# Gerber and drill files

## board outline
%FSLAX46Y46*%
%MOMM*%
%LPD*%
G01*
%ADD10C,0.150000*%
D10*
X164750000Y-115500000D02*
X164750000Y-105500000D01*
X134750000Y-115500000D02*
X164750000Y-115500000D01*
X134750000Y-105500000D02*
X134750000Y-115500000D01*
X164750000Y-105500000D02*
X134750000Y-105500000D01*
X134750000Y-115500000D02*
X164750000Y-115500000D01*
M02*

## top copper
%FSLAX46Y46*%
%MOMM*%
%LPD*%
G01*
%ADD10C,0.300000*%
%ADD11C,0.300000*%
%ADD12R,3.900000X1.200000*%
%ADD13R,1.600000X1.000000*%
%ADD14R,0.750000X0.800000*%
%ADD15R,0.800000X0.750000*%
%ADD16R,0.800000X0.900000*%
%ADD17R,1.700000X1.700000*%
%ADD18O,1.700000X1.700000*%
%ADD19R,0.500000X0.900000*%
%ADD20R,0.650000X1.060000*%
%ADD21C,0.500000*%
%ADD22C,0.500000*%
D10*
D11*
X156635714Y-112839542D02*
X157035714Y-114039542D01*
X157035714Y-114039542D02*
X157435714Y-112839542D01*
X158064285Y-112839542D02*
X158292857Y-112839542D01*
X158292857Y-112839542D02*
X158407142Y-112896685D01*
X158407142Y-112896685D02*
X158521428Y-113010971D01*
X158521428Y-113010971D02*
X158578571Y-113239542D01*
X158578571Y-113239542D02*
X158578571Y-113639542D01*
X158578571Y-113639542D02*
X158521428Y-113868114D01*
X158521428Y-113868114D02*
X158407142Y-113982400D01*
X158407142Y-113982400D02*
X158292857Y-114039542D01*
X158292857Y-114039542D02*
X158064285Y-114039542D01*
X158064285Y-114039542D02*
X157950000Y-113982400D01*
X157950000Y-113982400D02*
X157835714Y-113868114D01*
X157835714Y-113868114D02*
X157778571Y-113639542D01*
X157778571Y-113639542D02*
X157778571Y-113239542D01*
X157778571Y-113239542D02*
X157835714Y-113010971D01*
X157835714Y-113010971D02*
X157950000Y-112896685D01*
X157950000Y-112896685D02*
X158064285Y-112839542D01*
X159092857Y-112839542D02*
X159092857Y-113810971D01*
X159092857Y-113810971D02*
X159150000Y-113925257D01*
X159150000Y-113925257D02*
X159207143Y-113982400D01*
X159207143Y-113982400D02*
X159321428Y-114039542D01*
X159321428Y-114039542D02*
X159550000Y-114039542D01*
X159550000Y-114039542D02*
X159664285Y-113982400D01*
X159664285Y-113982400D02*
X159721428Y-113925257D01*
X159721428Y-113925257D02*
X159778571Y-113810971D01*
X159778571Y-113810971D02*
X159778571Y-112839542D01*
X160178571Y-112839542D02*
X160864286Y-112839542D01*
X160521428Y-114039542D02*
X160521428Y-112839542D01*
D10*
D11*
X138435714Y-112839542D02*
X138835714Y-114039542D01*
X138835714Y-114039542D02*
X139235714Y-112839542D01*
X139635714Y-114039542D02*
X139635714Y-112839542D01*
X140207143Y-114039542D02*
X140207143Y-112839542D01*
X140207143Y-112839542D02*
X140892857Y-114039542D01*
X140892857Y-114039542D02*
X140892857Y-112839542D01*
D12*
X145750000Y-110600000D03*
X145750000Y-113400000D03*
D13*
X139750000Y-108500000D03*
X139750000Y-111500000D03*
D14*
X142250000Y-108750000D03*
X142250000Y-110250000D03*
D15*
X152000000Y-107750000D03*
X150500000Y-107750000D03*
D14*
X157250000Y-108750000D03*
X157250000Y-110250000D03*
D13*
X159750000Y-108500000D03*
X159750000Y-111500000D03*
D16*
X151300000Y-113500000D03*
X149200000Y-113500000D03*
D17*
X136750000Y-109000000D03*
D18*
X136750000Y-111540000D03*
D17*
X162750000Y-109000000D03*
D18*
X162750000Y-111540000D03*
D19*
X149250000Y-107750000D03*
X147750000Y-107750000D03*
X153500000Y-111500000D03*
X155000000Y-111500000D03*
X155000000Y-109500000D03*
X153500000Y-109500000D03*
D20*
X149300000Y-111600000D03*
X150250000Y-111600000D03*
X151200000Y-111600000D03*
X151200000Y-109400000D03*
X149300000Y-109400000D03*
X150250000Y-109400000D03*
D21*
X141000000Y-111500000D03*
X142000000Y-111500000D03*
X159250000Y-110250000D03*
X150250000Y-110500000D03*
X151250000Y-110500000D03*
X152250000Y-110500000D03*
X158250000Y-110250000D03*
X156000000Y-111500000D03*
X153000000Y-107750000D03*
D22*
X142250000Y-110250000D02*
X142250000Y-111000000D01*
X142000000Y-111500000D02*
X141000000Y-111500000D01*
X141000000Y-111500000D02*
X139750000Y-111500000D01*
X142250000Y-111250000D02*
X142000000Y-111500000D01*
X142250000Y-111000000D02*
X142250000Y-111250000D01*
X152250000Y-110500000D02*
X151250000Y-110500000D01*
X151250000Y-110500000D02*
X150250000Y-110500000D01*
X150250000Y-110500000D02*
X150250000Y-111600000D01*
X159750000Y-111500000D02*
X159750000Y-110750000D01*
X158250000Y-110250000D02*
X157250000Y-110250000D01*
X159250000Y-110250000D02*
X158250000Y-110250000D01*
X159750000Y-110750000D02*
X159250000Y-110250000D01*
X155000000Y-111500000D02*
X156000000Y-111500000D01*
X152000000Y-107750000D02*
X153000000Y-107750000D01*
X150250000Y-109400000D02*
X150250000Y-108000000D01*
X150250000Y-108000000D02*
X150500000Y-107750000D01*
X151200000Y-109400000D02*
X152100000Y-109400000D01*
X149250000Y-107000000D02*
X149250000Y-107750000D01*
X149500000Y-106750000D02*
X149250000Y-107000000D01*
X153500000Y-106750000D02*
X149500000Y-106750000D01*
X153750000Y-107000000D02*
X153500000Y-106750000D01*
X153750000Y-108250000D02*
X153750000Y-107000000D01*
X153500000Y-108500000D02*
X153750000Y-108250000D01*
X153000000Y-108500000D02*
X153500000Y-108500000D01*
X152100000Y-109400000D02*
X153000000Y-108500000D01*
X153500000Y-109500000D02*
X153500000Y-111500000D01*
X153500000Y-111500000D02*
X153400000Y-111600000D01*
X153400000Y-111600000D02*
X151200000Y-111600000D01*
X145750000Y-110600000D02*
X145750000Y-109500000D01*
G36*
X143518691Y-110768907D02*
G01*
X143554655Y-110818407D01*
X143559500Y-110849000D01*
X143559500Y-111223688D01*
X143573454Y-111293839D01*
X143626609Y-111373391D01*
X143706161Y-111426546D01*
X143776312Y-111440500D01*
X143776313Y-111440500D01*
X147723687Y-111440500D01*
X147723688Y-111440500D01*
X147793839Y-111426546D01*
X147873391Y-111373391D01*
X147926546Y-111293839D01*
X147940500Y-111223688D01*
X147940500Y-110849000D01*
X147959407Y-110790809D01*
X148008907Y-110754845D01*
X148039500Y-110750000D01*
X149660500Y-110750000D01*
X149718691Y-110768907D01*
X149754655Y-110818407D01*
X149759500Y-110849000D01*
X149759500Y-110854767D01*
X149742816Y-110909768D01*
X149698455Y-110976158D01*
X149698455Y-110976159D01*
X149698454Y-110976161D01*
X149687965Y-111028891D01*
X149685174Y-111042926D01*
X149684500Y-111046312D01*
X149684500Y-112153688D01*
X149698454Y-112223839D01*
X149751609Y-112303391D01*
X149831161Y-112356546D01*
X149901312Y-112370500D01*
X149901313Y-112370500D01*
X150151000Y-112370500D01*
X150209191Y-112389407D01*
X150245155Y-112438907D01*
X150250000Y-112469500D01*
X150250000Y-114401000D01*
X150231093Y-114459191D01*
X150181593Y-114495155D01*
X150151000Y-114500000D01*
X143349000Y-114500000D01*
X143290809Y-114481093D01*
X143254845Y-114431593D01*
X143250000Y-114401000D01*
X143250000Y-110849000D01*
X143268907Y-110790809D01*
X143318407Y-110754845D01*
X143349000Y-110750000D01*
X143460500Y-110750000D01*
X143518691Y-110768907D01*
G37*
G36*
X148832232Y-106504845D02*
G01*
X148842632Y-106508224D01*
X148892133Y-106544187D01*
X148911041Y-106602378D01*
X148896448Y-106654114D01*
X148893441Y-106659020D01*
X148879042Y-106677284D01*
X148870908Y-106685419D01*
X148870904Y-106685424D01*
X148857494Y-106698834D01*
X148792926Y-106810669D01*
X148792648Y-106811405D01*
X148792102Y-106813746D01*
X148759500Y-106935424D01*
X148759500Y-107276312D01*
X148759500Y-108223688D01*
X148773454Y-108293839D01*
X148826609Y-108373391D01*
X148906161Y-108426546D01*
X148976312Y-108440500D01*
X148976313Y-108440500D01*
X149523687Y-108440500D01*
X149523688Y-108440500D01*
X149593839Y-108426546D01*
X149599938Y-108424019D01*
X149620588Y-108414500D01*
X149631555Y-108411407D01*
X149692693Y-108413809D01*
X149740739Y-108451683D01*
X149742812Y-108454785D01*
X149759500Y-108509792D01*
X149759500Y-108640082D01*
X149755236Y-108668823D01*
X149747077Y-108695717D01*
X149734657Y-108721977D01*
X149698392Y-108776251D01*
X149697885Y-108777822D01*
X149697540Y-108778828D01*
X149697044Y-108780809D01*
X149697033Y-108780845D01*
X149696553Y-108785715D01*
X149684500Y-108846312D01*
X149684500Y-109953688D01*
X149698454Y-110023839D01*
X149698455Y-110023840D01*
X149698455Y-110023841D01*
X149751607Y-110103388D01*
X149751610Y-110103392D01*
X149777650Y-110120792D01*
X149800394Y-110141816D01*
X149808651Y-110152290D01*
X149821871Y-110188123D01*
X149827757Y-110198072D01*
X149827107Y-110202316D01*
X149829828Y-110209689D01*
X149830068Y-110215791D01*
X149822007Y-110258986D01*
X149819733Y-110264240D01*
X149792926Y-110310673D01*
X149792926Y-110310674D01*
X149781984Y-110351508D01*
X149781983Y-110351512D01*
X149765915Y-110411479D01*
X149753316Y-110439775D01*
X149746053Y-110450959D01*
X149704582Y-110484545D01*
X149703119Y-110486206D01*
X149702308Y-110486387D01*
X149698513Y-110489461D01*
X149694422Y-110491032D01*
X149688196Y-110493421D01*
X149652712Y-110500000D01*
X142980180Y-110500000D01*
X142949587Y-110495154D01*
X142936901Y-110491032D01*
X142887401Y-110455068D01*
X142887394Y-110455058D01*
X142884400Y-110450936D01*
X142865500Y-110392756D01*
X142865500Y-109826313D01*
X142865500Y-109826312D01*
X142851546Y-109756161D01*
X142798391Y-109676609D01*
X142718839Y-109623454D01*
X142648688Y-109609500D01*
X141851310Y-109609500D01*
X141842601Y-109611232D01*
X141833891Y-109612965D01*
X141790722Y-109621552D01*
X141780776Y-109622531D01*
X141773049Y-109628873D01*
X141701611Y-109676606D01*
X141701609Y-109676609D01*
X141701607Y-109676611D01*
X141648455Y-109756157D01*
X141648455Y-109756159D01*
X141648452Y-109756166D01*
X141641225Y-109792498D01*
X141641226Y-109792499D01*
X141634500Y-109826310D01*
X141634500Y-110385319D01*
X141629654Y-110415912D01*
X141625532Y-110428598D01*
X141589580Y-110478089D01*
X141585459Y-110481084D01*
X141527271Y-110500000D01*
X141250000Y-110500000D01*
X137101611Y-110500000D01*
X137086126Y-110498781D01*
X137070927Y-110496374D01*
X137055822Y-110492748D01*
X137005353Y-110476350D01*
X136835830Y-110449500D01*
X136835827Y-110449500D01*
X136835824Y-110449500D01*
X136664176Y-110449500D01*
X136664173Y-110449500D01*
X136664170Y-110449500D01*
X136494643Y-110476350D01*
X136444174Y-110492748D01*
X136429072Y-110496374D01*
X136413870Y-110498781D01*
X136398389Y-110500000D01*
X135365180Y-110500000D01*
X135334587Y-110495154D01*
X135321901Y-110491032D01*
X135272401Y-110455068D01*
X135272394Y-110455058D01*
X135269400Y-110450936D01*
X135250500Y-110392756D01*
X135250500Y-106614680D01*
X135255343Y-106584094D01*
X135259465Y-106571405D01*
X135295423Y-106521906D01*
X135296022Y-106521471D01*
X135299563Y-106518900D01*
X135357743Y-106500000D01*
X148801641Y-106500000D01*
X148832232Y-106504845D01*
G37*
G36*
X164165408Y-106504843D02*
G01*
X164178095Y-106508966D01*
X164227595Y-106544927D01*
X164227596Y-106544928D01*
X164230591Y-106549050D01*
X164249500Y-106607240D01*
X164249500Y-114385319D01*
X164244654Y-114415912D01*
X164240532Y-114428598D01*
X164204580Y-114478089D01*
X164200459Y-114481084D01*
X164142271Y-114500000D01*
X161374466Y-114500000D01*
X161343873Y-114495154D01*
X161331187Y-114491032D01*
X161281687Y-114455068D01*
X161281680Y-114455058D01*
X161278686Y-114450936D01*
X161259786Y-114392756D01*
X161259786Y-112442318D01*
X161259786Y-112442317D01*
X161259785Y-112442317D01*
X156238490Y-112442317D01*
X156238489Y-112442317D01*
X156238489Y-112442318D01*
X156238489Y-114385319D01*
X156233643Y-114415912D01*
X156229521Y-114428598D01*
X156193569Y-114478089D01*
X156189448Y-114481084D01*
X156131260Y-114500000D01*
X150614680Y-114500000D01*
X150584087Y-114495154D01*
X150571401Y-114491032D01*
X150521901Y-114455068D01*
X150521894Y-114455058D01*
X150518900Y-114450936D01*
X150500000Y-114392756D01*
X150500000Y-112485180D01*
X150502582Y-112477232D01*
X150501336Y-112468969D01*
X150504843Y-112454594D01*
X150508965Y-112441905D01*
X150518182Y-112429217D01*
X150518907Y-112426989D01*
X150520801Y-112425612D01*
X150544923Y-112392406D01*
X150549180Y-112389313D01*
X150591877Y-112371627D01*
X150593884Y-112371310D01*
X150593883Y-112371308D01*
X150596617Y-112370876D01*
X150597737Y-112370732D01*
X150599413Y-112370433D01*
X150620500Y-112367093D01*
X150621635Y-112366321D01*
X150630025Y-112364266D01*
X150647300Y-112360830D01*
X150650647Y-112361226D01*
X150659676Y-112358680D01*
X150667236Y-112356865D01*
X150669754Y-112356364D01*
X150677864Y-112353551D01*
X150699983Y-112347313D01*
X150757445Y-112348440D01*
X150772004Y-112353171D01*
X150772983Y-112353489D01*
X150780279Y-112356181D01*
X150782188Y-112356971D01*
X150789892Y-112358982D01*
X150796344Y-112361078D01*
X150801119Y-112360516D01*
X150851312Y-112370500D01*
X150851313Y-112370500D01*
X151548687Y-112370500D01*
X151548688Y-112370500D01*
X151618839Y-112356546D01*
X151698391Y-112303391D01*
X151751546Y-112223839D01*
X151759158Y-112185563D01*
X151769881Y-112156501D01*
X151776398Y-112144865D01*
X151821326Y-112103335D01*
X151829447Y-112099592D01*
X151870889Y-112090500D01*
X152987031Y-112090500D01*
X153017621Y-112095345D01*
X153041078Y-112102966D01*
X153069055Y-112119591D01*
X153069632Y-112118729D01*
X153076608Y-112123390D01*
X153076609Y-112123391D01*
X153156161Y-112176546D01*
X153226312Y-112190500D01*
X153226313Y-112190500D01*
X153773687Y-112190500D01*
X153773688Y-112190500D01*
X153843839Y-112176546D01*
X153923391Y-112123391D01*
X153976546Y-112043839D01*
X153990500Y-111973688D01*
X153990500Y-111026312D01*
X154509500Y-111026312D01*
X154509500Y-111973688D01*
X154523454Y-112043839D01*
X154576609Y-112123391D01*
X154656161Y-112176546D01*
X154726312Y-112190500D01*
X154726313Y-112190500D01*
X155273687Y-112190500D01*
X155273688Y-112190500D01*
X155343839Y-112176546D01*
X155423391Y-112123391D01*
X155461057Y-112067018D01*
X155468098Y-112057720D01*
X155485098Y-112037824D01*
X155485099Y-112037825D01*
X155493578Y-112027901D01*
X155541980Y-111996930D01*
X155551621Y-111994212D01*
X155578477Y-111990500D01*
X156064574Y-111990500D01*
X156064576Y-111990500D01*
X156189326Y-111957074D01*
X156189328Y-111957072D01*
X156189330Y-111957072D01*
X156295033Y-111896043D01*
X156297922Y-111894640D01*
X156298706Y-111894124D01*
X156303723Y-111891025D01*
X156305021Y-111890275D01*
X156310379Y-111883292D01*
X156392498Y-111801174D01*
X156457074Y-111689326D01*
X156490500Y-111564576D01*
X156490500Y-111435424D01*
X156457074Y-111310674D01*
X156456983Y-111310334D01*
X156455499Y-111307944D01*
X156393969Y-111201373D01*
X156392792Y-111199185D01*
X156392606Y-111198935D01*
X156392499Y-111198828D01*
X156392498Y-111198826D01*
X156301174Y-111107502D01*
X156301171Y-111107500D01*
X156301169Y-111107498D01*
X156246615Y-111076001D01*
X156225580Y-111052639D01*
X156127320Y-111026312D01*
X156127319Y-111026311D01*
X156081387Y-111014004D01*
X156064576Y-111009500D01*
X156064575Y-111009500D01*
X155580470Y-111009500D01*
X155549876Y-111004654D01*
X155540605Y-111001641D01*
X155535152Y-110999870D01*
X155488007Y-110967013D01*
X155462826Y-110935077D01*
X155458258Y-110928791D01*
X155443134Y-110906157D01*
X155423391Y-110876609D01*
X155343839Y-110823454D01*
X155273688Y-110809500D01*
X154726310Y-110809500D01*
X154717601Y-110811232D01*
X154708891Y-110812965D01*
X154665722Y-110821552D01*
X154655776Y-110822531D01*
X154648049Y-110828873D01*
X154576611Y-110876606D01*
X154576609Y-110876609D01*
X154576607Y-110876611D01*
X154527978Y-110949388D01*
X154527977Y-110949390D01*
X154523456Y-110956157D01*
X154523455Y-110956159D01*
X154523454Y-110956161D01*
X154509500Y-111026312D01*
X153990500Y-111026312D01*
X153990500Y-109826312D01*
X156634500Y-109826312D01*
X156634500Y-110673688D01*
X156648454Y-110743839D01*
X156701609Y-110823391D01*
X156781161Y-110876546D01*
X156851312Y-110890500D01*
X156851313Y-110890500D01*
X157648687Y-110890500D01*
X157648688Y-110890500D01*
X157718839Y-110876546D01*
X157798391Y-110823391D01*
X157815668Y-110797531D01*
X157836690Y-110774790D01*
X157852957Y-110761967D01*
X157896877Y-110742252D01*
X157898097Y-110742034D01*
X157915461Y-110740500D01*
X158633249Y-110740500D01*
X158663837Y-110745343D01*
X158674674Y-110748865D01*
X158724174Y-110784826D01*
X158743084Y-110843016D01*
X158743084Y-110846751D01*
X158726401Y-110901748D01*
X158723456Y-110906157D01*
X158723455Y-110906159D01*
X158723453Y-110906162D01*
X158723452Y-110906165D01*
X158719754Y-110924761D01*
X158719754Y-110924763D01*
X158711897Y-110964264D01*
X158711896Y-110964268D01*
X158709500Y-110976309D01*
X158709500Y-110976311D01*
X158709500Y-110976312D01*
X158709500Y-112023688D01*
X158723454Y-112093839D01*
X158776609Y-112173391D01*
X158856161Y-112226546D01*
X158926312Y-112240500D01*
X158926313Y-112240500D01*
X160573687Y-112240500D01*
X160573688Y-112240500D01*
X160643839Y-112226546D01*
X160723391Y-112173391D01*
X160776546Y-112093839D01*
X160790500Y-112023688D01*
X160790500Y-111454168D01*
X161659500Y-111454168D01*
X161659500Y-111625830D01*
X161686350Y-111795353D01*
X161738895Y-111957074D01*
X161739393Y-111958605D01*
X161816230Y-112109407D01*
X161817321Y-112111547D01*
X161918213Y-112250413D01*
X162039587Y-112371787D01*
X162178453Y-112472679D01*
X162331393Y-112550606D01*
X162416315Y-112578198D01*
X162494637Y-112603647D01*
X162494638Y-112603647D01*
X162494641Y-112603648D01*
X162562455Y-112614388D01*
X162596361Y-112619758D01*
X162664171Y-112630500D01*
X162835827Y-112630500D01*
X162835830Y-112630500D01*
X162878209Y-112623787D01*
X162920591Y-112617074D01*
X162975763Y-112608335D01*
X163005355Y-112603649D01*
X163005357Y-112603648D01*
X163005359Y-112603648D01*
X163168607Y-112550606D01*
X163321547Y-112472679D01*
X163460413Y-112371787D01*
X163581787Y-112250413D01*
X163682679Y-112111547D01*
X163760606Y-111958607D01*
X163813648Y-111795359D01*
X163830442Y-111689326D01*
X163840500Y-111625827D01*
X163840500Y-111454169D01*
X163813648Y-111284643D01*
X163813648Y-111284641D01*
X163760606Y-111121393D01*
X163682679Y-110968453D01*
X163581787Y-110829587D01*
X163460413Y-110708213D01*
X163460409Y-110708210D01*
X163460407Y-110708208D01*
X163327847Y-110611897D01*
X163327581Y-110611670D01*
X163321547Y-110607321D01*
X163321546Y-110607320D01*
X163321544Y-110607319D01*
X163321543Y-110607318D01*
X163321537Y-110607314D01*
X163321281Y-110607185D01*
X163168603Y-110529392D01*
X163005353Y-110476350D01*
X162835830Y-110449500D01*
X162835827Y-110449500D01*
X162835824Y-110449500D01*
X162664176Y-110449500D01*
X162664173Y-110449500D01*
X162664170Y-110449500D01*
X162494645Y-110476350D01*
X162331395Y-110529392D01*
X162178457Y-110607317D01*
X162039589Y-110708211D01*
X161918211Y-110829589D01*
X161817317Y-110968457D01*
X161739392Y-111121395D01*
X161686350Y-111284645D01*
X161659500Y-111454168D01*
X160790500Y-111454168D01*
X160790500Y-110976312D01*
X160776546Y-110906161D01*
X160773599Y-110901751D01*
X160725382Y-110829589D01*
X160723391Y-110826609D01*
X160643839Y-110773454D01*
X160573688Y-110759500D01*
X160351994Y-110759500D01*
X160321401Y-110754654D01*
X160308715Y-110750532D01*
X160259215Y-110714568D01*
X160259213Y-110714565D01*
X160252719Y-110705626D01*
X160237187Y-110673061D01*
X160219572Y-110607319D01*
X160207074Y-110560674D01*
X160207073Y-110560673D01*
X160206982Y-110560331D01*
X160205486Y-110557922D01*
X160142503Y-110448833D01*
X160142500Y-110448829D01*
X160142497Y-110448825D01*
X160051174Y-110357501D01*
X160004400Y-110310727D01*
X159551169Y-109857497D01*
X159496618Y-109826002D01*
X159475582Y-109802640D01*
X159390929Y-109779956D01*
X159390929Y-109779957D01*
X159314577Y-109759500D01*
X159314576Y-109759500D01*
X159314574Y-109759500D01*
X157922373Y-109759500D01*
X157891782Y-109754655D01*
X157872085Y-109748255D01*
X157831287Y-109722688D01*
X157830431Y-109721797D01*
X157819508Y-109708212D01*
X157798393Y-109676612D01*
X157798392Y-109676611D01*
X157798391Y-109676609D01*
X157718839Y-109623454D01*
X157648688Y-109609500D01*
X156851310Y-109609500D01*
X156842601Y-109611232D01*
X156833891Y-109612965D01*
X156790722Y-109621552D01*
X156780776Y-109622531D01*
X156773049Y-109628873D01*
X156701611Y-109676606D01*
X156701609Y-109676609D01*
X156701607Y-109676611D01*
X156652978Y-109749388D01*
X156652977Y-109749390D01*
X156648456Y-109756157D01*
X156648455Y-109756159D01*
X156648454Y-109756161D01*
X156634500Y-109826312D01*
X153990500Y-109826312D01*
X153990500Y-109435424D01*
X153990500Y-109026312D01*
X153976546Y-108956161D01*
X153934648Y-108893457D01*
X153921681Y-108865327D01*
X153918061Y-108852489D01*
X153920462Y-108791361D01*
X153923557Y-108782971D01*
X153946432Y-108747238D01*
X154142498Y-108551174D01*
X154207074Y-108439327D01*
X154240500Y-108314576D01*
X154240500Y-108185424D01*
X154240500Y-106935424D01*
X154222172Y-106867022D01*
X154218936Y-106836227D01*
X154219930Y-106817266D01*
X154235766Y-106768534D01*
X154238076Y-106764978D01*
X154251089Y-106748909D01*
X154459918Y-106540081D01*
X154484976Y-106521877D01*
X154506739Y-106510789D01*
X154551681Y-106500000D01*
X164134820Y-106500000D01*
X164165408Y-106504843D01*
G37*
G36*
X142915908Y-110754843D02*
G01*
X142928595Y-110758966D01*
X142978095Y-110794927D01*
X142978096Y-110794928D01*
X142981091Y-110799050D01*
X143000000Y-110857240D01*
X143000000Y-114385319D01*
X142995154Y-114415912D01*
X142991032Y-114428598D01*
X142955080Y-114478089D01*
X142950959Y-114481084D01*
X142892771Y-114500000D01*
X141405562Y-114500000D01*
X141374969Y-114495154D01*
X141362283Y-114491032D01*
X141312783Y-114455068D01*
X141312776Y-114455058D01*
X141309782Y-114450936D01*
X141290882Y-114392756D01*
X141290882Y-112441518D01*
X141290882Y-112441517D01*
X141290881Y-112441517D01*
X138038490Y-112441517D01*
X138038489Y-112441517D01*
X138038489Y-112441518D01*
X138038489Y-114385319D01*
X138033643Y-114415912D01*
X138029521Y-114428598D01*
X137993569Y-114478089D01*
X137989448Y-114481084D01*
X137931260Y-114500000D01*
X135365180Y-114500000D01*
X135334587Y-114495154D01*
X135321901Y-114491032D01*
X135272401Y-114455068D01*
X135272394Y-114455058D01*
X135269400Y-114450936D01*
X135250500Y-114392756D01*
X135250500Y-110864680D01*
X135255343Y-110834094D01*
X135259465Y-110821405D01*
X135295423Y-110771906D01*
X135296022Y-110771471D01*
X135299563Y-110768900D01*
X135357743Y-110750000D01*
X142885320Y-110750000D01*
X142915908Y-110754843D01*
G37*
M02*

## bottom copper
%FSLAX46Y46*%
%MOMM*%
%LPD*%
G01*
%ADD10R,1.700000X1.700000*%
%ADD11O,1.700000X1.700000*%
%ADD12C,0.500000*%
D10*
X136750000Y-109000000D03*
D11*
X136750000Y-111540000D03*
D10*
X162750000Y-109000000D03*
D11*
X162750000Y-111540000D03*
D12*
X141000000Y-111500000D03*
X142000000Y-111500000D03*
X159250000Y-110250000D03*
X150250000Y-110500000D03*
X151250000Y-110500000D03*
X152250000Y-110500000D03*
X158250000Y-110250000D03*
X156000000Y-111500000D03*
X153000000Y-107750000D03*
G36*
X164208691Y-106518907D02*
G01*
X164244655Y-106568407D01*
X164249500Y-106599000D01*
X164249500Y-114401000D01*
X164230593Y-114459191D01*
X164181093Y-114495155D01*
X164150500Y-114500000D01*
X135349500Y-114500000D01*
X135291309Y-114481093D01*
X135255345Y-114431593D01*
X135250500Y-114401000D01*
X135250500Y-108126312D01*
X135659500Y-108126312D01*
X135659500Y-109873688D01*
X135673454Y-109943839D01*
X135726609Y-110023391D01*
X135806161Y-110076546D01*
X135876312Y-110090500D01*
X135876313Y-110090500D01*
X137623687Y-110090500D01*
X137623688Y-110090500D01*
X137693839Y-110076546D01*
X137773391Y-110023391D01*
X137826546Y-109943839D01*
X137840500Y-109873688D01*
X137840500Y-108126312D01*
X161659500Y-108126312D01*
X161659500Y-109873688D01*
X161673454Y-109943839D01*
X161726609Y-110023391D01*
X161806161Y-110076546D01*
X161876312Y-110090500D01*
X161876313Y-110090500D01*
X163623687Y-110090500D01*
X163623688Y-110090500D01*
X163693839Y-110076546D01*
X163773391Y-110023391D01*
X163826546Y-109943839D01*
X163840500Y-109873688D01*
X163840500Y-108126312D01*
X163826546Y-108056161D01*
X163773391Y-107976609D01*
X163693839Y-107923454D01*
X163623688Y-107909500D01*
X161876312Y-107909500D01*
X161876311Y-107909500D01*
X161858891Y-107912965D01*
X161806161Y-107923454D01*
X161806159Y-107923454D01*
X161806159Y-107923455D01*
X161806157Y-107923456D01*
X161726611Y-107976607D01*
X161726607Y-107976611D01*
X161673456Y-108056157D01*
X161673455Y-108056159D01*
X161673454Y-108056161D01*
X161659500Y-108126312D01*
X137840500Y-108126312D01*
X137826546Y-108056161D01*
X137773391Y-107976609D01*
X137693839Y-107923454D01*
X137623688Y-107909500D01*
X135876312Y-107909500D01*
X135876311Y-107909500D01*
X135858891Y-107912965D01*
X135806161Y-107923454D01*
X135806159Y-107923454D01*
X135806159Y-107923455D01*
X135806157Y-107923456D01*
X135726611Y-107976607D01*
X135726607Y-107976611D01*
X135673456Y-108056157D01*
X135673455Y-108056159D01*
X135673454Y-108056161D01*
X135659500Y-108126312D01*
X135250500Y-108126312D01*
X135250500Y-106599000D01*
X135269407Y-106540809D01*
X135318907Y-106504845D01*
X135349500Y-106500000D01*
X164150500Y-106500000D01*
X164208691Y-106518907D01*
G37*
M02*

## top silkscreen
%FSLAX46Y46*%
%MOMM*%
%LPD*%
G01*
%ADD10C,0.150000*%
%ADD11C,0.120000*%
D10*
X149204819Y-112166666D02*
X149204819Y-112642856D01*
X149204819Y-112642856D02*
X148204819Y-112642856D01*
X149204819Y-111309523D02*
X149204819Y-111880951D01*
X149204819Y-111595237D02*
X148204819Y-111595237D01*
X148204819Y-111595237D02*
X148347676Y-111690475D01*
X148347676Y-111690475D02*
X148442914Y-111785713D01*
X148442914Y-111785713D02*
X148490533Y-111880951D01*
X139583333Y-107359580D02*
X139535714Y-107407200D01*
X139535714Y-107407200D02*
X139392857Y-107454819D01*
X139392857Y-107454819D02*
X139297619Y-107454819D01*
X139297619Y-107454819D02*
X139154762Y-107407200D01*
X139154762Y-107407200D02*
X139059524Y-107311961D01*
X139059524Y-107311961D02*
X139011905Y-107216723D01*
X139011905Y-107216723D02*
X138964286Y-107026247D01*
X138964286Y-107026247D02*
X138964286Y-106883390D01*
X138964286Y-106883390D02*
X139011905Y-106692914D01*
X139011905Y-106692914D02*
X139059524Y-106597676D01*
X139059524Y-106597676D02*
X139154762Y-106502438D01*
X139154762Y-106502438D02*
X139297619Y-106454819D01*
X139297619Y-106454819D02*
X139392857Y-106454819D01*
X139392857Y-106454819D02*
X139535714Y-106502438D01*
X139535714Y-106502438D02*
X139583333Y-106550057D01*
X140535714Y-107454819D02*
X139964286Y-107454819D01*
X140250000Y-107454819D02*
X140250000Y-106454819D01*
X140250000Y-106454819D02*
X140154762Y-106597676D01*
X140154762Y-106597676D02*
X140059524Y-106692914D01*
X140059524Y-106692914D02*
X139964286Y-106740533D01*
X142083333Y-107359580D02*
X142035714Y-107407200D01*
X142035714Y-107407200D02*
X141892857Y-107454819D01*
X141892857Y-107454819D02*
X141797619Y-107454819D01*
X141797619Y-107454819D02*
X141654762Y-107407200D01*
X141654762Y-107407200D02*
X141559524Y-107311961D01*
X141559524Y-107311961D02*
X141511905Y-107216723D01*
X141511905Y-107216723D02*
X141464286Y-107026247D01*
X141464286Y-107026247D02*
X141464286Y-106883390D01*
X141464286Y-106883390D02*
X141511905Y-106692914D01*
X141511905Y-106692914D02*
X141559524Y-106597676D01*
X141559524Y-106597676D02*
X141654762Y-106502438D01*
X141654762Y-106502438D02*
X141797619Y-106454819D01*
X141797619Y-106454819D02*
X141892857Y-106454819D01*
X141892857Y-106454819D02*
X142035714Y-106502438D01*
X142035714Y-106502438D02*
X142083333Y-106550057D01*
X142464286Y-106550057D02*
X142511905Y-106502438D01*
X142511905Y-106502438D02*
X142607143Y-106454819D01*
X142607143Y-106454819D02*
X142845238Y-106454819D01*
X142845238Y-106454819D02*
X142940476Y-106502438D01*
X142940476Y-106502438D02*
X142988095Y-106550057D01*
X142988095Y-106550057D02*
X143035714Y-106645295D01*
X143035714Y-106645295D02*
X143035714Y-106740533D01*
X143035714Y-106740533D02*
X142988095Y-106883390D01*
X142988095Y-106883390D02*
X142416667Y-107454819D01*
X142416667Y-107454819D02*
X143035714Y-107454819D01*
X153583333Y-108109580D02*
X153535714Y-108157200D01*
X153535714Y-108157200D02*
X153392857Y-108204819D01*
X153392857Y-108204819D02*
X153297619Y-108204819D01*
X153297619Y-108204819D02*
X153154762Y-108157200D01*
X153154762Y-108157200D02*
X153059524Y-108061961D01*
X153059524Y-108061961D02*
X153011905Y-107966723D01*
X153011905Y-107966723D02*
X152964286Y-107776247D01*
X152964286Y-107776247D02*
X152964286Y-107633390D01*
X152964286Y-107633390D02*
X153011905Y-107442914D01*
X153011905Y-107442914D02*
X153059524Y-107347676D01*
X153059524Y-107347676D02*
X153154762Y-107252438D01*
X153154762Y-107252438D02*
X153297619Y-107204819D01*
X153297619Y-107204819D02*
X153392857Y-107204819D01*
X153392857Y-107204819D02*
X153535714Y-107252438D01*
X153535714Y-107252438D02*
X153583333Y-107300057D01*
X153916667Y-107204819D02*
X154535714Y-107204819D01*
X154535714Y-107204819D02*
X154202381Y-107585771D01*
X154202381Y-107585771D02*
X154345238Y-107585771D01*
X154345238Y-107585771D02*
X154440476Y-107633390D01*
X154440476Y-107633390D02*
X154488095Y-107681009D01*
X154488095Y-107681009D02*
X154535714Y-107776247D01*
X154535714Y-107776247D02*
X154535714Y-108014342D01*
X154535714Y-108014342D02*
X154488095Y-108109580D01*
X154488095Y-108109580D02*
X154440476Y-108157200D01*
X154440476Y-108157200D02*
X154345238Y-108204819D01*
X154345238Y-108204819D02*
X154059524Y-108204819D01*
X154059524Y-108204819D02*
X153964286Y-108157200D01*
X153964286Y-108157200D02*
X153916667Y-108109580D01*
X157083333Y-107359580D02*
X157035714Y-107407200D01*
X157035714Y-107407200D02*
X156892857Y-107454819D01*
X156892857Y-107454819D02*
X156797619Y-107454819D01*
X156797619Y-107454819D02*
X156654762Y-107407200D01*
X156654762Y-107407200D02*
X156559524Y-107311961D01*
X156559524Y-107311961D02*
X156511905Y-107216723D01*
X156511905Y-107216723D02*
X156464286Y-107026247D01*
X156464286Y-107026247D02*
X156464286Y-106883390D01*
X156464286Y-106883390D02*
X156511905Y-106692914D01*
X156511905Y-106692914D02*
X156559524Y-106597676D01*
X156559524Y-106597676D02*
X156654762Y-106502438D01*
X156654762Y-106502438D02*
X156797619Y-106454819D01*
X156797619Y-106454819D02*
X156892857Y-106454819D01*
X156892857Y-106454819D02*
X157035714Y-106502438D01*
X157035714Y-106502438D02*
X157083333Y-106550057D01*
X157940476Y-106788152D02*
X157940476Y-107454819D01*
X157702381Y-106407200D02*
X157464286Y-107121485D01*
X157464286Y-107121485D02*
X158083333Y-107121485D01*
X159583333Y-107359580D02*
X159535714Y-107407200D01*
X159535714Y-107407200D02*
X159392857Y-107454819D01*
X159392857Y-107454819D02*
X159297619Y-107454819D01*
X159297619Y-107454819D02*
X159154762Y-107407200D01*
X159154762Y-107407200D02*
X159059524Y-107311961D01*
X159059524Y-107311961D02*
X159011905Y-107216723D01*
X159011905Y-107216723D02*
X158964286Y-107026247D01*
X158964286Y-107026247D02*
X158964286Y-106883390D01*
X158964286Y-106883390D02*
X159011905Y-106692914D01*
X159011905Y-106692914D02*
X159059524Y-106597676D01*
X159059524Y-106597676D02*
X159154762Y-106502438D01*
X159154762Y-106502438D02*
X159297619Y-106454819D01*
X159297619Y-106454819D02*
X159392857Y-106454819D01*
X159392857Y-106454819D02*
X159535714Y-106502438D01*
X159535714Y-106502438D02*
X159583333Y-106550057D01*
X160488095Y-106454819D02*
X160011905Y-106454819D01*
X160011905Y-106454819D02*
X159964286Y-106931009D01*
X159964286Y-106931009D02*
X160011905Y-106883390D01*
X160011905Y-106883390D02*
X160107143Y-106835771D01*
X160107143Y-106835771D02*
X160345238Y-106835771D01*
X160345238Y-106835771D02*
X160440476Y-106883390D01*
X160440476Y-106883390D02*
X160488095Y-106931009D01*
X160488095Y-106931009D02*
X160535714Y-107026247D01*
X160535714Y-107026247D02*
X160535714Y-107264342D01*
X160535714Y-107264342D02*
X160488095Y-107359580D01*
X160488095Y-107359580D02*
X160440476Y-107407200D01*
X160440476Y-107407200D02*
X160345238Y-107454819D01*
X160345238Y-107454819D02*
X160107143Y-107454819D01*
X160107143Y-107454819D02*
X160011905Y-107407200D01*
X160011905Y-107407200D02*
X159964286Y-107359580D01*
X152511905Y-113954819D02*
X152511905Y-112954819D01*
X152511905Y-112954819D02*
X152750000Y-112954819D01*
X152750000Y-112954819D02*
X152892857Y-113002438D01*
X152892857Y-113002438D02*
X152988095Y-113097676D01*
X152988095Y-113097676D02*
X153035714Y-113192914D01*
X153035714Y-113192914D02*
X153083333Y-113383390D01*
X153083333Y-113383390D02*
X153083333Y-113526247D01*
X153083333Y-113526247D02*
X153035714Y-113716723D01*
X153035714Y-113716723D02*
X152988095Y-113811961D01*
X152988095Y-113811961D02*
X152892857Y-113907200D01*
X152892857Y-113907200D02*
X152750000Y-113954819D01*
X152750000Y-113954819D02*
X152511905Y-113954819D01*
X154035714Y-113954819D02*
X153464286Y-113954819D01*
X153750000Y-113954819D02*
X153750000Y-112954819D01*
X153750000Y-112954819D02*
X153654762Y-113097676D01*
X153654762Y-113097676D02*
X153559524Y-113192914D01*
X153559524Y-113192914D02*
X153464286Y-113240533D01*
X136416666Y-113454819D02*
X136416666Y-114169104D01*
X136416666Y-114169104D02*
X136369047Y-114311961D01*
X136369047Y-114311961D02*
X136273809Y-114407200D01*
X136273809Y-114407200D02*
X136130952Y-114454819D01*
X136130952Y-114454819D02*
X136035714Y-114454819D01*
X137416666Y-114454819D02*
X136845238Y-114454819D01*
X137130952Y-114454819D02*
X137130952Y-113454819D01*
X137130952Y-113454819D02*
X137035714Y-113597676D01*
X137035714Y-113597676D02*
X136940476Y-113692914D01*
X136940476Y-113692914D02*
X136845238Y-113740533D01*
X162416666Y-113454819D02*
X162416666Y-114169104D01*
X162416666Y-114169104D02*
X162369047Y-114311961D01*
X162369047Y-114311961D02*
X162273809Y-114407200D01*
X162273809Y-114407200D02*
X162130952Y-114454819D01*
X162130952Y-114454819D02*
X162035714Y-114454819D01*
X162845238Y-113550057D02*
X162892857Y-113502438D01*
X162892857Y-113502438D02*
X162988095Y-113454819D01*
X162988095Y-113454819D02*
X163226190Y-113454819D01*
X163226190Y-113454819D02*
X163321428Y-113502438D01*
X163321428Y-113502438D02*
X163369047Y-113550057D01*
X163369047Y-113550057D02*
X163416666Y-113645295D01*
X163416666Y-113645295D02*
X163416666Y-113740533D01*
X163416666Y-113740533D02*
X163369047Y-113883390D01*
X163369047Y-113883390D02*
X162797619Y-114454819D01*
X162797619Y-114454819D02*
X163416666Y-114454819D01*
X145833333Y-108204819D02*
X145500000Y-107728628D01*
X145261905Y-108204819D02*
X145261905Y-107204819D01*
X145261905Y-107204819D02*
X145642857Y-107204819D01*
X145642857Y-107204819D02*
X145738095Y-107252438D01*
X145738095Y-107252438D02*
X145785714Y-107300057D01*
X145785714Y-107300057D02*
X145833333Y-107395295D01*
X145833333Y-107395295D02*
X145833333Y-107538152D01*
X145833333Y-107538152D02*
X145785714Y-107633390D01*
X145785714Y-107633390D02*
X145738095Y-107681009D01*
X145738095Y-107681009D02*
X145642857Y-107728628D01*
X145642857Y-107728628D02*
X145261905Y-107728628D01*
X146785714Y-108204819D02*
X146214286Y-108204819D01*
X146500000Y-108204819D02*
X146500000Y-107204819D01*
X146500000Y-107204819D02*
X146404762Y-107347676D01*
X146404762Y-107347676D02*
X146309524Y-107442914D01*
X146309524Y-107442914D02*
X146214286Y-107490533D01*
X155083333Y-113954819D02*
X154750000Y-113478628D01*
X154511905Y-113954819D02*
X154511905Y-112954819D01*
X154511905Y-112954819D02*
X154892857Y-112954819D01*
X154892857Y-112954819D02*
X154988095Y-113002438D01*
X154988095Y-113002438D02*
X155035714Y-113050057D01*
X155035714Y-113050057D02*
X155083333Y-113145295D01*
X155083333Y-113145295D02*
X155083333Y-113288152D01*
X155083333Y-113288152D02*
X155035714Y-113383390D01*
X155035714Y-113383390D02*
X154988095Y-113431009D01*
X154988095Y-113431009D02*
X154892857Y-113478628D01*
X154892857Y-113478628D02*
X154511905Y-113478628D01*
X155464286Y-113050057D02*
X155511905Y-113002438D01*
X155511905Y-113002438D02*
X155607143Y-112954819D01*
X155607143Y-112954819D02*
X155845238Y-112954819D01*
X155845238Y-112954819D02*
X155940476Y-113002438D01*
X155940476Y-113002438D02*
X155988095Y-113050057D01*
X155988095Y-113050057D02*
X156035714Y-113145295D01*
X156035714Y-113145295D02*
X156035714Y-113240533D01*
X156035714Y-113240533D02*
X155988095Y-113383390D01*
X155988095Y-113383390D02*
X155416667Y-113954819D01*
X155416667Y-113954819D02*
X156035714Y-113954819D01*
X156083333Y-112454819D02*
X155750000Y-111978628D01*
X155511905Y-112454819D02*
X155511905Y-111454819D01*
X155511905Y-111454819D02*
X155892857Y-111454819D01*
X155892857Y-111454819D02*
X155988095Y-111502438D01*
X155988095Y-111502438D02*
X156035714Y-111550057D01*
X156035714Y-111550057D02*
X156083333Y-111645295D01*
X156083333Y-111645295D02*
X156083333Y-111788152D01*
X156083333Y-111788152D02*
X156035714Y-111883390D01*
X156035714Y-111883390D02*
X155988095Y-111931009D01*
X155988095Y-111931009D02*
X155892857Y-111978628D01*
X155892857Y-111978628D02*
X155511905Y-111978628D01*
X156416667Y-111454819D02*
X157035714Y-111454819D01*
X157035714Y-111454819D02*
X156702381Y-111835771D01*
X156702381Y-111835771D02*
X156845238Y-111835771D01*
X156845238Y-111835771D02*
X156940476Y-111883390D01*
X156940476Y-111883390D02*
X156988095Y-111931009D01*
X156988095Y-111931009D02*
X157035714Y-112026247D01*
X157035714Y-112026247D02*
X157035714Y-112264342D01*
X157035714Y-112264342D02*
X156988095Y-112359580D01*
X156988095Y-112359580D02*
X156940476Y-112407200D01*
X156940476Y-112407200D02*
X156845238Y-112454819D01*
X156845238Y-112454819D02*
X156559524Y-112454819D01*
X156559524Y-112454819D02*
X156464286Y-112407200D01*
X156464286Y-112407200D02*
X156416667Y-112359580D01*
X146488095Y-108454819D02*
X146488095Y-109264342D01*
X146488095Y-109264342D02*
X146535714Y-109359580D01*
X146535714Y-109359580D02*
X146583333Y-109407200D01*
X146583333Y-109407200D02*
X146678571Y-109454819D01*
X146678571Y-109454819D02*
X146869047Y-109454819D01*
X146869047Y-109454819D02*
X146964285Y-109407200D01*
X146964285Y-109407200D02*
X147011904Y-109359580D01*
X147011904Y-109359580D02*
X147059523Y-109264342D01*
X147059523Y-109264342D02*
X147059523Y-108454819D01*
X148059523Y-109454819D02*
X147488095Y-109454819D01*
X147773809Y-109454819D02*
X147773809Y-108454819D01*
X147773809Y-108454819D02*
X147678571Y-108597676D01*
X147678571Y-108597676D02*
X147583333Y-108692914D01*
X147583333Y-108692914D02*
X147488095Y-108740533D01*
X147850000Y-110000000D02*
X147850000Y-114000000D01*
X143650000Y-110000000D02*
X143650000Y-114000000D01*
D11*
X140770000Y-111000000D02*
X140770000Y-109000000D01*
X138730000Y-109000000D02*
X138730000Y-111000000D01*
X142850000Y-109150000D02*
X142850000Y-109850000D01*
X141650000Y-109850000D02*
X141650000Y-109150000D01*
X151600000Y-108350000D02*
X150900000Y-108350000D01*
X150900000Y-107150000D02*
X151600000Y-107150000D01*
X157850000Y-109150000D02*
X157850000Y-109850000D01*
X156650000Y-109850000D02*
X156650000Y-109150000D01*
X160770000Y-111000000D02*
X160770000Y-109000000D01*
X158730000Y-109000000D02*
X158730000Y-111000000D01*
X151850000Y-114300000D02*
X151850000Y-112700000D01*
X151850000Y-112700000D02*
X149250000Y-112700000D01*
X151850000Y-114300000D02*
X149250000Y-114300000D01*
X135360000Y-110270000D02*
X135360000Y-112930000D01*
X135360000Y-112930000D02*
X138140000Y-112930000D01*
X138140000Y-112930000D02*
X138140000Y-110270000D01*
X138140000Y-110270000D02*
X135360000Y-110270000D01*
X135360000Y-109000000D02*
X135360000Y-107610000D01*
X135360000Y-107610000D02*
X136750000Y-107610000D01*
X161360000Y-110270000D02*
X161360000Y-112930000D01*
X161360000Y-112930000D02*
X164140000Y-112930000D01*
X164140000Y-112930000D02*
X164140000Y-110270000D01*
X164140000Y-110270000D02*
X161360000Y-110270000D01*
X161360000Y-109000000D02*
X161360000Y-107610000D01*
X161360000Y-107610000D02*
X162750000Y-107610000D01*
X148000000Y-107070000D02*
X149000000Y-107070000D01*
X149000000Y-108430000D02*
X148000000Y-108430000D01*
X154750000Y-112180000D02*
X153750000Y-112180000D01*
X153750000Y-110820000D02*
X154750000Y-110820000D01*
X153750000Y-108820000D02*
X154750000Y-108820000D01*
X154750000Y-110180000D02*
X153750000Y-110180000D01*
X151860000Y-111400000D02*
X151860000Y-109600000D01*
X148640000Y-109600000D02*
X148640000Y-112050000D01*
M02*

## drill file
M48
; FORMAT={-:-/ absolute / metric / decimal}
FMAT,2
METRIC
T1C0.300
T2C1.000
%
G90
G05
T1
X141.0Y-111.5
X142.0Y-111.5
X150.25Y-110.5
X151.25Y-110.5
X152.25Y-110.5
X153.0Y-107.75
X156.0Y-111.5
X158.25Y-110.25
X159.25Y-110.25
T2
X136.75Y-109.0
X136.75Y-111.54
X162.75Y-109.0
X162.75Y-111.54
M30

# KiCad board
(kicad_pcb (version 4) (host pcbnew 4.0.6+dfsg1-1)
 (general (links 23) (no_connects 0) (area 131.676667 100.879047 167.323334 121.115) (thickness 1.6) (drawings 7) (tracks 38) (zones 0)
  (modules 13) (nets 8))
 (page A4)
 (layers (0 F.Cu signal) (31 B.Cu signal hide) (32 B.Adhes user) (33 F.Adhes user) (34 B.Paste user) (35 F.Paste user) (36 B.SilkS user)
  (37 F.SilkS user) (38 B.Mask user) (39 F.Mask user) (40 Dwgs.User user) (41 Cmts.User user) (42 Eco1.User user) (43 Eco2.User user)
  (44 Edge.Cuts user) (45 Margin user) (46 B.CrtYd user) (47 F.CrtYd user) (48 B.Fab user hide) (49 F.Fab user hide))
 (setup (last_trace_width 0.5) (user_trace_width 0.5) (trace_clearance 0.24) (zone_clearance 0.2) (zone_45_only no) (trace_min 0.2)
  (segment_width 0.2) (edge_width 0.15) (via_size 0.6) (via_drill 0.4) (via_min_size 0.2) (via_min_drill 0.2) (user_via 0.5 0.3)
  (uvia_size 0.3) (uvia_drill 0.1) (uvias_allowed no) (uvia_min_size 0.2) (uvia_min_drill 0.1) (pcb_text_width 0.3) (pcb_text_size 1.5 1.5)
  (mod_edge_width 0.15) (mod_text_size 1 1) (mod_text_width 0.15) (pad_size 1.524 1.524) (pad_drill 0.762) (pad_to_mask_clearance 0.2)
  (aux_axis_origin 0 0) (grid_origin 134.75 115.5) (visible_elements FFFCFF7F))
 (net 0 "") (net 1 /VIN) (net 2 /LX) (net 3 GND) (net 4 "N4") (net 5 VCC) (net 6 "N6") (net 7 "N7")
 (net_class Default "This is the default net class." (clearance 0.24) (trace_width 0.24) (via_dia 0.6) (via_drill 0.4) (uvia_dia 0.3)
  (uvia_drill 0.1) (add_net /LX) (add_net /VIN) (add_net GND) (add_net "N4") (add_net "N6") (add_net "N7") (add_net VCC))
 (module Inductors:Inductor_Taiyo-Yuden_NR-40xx (layer F.Cu) (at 145.75 112 270)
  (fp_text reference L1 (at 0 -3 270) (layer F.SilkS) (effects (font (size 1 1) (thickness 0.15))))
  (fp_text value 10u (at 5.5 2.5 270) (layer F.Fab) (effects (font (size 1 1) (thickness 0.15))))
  (fp_line (start -2 -2.1) (end 2 -2.1) (layer F.SilkS) (width 0.15))
  (fp_line (start -2 2.1) (end 2 2.1) (layer F.SilkS) (width 0.15))
  (pad 1 smd rect (at -1.4 0 270) (size 1.2 3.9) (layers F.Cu F.Paste F.Mask) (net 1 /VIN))
  (pad 2 smd rect (at 1.4 0 270) (size 1.2 3.9) (layers F.Cu F.Paste F.Mask) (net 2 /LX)))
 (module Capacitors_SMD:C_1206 (layer F.Cu) (at 139.75 110 270)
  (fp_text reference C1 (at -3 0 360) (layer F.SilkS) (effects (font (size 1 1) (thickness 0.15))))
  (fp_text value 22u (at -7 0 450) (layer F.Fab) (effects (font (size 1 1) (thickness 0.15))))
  (fp_line (start 1 -1.02) (end -1 -1.02) (layer F.SilkS) (width 0.12))
  (fp_line (start -1 1.02) (end 1 1.02) (layer F.SilkS) (width 0.12))
  (pad 1 smd rect (at -1.5 0 270) (size 1 1.6) (layers F.Cu F.Paste F.Mask) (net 1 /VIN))
  (pad 2 smd rect (at 1.5 0 270) (size 1 1.6) (layers F.Cu F.Paste F.Mask) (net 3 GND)))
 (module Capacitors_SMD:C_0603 (layer F.Cu) (at 142.25 109.5 270)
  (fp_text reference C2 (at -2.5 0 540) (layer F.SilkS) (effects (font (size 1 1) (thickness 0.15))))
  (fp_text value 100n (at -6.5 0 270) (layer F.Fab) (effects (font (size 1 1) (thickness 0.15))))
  (fp_line (start -0.35 -0.6) (end 0.35 -0.6) (layer F.SilkS) (width 0.12))
  (fp_line (start 0.35 0.6) (end -0.35 0.6) (layer F.SilkS) (width 0.12))
  (pad 1 smd rect (at -0.75 0 270) (size 0.8 0.75) (layers F.Cu F.Paste F.Mask) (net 1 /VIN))
  (pad 2 smd rect (at 0.75 0 270) (size 0.8 0.75) (layers F.Cu F.Paste F.Mask) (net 3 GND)))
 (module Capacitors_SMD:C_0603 (layer F.Cu) (at 151.25 107.75 180)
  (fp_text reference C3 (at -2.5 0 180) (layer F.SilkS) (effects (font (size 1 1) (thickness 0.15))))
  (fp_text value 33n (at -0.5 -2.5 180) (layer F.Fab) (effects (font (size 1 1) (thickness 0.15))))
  (fp_line (start -0.35 -0.6) (end 0.35 -0.6) (layer F.SilkS) (width 0.12))
  (fp_line (start 0.35 0.6) (end -0.35 0.6) (layer F.SilkS) (width 0.12))
  (pad 1 smd rect (at -0.75 0 180) (size 0.8 0.75) (layers F.Cu F.Paste F.Mask) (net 3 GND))
  (pad 2 smd rect (at 0.75 0 180) (size 0.8 0.75) (layers F.Cu F.Paste F.Mask) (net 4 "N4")))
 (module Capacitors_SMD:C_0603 (layer F.Cu) (at 157.25 109.5 270)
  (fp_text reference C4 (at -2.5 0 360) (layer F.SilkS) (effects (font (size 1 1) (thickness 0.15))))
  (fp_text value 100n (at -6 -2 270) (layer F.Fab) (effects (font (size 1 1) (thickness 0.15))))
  (fp_line (start -0.35 -0.6) (end 0.35 -0.6) (layer F.SilkS) (width 0.12))
  (fp_line (start 0.35 0.6) (end -0.35 0.6) (layer F.SilkS) (width 0.12))
  (pad 1 smd rect (at -0.75 0 270) (size 0.8 0.75) (layers F.Cu F.Paste F.Mask) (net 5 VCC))
  (pad 2 smd rect (at 0.75 0 270) (size 0.8 0.75) (layers F.Cu F.Paste F.Mask) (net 3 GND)))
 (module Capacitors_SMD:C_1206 (layer F.Cu) (at 159.75 110 270)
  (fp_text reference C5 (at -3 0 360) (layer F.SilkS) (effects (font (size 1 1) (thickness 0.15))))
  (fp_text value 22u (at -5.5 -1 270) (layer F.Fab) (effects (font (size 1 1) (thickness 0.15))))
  (fp_line (start 1 -1.02) (end -1 -1.02) (layer F.SilkS) (width 0.12))
  (fp_line (start -1 1.02) (end 1 1.02) (layer F.SilkS) (width 0.12))
  (pad 1 smd rect (at -1.5 0 270) (size 1 1.6) (layers F.Cu F.Paste F.Mask) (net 5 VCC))
  (pad 2 smd rect (at 1.5 0 270) (size 1 1.6) (layers F.Cu F.Paste F.Mask) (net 3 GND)))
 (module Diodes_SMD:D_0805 (layer F.Cu) (at 150.25 113.5 180)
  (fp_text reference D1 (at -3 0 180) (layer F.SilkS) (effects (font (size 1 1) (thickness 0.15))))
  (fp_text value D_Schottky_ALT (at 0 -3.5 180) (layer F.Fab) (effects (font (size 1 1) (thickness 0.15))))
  (fp_line (start -1.6 -0.8) (end -1.6 0.8) (layer F.SilkS) (width 0.12))
  (fp_line (start -1.6 0.8) (end 1 0.8) (layer F.SilkS) (width 0.12))
  (fp_line (start -1.6 -0.8) (end 1 -0.8) (layer F.SilkS) (width 0.12))
  (pad 1 smd rect (at -1.05 0 180) (size 0.8 0.9) (layers F.Cu F.Paste F.Mask) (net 5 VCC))
  (pad 2 smd rect (at 1.05 0 180) (size 0.8 0.9) (layers F.Cu F.Paste F.Mask) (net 2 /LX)))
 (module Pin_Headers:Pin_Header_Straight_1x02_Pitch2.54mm (layer F.Cu) (at 136.75 109)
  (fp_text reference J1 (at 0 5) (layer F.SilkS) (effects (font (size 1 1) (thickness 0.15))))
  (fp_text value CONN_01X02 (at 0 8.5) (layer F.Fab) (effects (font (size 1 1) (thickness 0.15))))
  (fp_line (start -1.39 1.27) (end -1.39 3.93) (layer F.SilkS) (width 0.12))
  (fp_line (start -1.39 3.93) (end 1.39 3.93) (layer F.SilkS) (width 0.12))
  (fp_line (start 1.39 3.93) (end 1.39 1.27) (layer F.SilkS) (width 0.12))
  (fp_line (start 1.39 1.27) (end -1.39 1.27) (layer F.SilkS) (width 0.12))
  (fp_line (start -1.39 0) (end -1.39 -1.39) (layer F.SilkS) (width 0.12))
  (fp_line (start -1.39 -1.39) (end 0 -1.39) (layer F.SilkS) (width 0.12))
  (pad 1 thru_hole rect (at 0 0) (size 1.7 1.7) (drill 1) (layers *.Cu *.Mask) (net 1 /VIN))
  (pad 2 thru_hole oval (at 0 2.54) (size 1.7 1.7) (drill 1) (layers *.Cu *.Mask) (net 3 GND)))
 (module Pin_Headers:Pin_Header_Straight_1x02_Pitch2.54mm (layer F.Cu) (at 162.75 109)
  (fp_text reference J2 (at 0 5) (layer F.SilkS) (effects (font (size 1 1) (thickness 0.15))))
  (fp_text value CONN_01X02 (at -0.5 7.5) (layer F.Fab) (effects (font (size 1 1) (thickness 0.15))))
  (fp_line (start -1.39 1.27) (end -1.39 3.93) (layer F.SilkS) (width 0.12))
  (fp_line (start -1.39 3.93) (end 1.39 3.93) (layer F.SilkS) (width 0.12))
  (fp_line (start 1.39 3.93) (end 1.39 1.27) (layer F.SilkS) (width 0.12))
  (fp_line (start 1.39 1.27) (end -1.39 1.27) (layer F.SilkS) (width 0.12))
  (fp_line (start -1.39 0) (end -1.39 -1.39) (layer F.SilkS) (width 0.12))
  (fp_line (start -1.39 -1.39) (end 0 -1.39) (layer F.SilkS) (width 0.12))
  (pad 1 thru_hole rect (at 0 0) (size 1.7 1.7) (drill 1) (layers *.Cu *.Mask) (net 5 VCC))
  (pad 2 thru_hole oval (at 0 2.54) (size 1.7 1.7) (drill 1) (layers *.Cu *.Mask) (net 3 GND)))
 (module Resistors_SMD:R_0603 (layer F.Cu) (at 148.5 107.75 180)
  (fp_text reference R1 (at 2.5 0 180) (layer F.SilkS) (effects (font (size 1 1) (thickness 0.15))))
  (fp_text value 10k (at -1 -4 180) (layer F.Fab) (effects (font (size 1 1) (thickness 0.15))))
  (fp_line (start 0.5 0.68) (end -0.5 0.68) (layer F.SilkS) (width 0.12))
  (fp_line (start -0.5 -0.68) (end 0.5 -0.68) (layer F.SilkS) (width 0.12))
  (pad 1 smd rect (at -0.75 0 180) (size 0.5 0.9) (layers F.Cu F.Paste F.Mask) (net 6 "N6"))
  (pad 2 smd rect (at 0.75 0 180) (size 0.5 0.9) (layers F.Cu F.Paste F.Mask) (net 1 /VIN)))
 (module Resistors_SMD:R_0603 (layer F.Cu) (at 154.25 111.5)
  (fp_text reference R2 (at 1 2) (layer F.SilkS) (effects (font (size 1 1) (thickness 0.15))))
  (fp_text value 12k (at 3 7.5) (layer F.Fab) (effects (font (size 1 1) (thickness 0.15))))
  (fp_line (start 0.5 0.68) (end -0.5 0.68) (layer F.SilkS) (width 0.12))
  (fp_line (start -0.5 -0.68) (end 0.5 -0.68) (layer F.SilkS) (width 0.12))
  (pad 1 smd rect (at -0.75 0) (size 0.5 0.9) (layers F.Cu F.Paste F.Mask) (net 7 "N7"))
  (pad 2 smd rect (at 0.75 0) (size 0.5 0.9) (layers F.Cu F.Paste F.Mask) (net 3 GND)))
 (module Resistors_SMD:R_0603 (layer F.Cu) (at 154.25 109.5 180)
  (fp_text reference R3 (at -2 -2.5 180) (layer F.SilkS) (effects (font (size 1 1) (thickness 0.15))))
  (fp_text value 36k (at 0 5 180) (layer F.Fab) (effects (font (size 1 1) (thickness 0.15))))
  (fp_line (start 0.5 0.68) (end -0.5 0.68) (layer F.SilkS) (width 0.12))
  (fp_line (start -0.5 -0.68) (end 0.5 -0.68) (layer F.SilkS) (width 0.12))
  (pad 1 smd rect (at -0.75 0 180) (size 0.5 0.9) (layers F.Cu F.Paste F.Mask) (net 5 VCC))
  (pad 2 smd rect (at 0.75 0 180) (size 0.5 0.9) (layers F.Cu F.Paste F.Mask) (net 7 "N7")))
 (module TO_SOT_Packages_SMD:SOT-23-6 (layer F.Cu) (at 150.25 110.5 90)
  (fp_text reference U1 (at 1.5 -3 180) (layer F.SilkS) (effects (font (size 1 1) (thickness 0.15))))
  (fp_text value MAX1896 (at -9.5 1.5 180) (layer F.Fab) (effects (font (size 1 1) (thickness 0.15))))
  (fp_line (start -0.9 1.61) (end 0.9 1.61) (layer F.SilkS) (width 0.12))
  (fp_line (start 0.9 -1.61) (end -1.55 -1.61) (layer F.SilkS) (width 0.12))
  (pad 1 smd rect (at -1.1 -0.95 90) (size 1.06 0.65) (layers F.Cu F.Paste F.Mask) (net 2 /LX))
  (pad 2 smd rect (at -1.1 0 90) (size 1.06 0.65) (layers F.Cu F.Paste F.Mask) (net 3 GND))
  (pad 3 smd rect (at -1.1 0.95 90) (size 1.06 0.65) (layers F.Cu F.Paste F.Mask) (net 7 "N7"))
  (pad 4 smd rect (at 1.1 0.95 90) (size 1.06 0.65) (layers F.Cu F.Paste F.Mask) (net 6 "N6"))
  (pad 6 smd rect (at 1.1 -0.95 90) (size 1.06 0.65) (layers F.Cu F.Paste F.Mask) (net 1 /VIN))
  (pad 5 smd rect (at 1.1 0 90) (size 1.06 0.65) (layers F.Cu F.Paste F.Mask) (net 4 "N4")))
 (gr_line (start 164.75 115.5) (end 164.75 105.5) (angle 90) (layer Edge.Cuts) (width 0.15))
 (gr_line (start 134.75 115.5) (end 164.75 115.5) (angle 90) (layer Edge.Cuts) (width 0.15))
 (gr_line (start 134.75 105.5) (end 134.75 115.5) (angle 90) (layer Edge.Cuts) (width 0.15))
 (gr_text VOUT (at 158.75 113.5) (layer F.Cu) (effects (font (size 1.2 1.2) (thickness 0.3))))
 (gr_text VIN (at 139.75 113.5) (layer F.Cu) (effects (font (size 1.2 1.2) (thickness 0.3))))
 (gr_line (start 164.75 105.5) (end 134.75 105.5) (angle 90) (layer Edge.Cuts) (width 0.15))
 (gr_line (start 134.75 115.5) (end 164.75 115.5) (angle 90) (layer Edge.Cuts) (width 0.15))
 (via (at 141 111.5) (size 0.5) (drill 0.3) (layers F.Cu B.Cu) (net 3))
 (segment (start 142.25 110.25) (end 142.25 111) (width 0.5) (layer F.Cu) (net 3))
 (via (at 142 111.5) (size 0.5) (drill 0.3) (layers F.Cu B.Cu) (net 3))
 (segment (start 142 111.5) (end 141 111.5) (width 0.5) (layer F.Cu) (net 3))
 (segment (start 141 111.5) (end 139.75 111.5) (width 0.5) (layer F.Cu) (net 3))
 (segment (start 142.25 111.25) (end 142 111.5) (width 0.5) (layer F.Cu) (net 3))
 (segment (start 142.25 111) (end 142.25 111.25) (width 0.5) (layer F.Cu) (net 3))
 (via (at 159.25 110.25) (size 0.5) (drill 0.3) (layers F.Cu B.Cu) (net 3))
 (segment (start 152.25 110.5) (end 151.25 110.5) (width 0.5) (layer F.Cu) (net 3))
 (segment (start 151.25 110.5) (end 150.25 110.5) (width 0.5) (layer F.Cu) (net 3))
 (via (at 150.25 110.5) (size 0.5) (drill 0.3) (layers F.Cu B.Cu) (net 3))
 (segment (start 150.25 110.5) (end 150.25 111.6) (width 0.5) (layer F.Cu) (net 3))
 (via (at 151.25 110.5) (size 0.5) (drill 0.3) (layers F.Cu B.Cu) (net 3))
 (via (at 152.25 110.5) (size 0.5) (drill 0.3) (layers F.Cu B.Cu) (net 3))
 (segment (start 159.75 111.5) (end 159.75 110.75) (width 0.5) (layer F.Cu) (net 3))
 (via (at 158.25 110.25) (size 0.5) (drill 0.3) (layers F.Cu B.Cu) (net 3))
 (segment (start 158.25 110.25) (end 157.25 110.25) (width 0.5) (layer F.Cu) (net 3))
 (segment (start 159.25 110.25) (end 158.25 110.25) (width 0.5) (layer F.Cu) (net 3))
 (segment (start 159.75 110.75) (end 159.25 110.25) (width 0.5) (layer F.Cu) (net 3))
 (segment (start 155 111.5) (end 156 111.5) (width 0.5) (layer F.Cu) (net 3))
 (via (at 156 111.5) (size 0.5) (drill 0.3) (layers F.Cu B.Cu) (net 3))
 (segment (start 152 107.75) (end 153 107.75) (width 0.5) (layer F.Cu) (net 3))
 (via (at 153 107.75) (size 0.5) (drill 0.3) (layers F.Cu B.Cu) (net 3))
 (segment (start 150.25 109.4) (end 150.25 108) (width 0.5) (layer F.Cu) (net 4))
 (segment (start 150.25 108) (end 150.5 107.75) (width 0.5) (layer F.Cu) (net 4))
 (segment (start 151.2 109.4) (end 152.1 109.4) (width 0.5) (layer F.Cu) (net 6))
 (segment (start 149.25 107) (end 149.25 107.75) (width 0.5) (layer F.Cu) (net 6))
 (segment (start 149.5 106.75) (end 149.25 107) (width 0.5) (layer F.Cu) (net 6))
 (segment (start 153.5 106.75) (end 149.5 106.75) (width 0.5) (layer F.Cu) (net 6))
 (segment (start 153.75 107) (end 153.5 106.75) (width 0.5) (layer F.Cu) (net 6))
 (segment (start 153.75 108.25) (end 153.75 107) (width 0.5) (layer F.Cu) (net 6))
 (segment (start 153.5 108.5) (end 153.75 108.25) (width 0.5) (layer F.Cu) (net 6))
 (segment (start 153 108.5) (end 153.5 108.5) (width 0.5) (layer F.Cu) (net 6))
 (segment (start 152.1 109.4) (end 153 108.5) (width 0.5) (layer F.Cu) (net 6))
 (segment (start 153.5 109.5) (end 153.5 111.5) (width 0.5) (layer F.Cu) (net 7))
 (segment (start 153.5 111.5) (end 153.4 111.6) (width 0.5) (layer F.Cu) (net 7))
 (segment (start 153.4 111.6) (end 151.2 111.6) (width 0.5) (layer F.Cu) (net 7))
 (segment (start 145.75 110.6) (end 145.75 109.5) (width 0.5) (layer F.Cu) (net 1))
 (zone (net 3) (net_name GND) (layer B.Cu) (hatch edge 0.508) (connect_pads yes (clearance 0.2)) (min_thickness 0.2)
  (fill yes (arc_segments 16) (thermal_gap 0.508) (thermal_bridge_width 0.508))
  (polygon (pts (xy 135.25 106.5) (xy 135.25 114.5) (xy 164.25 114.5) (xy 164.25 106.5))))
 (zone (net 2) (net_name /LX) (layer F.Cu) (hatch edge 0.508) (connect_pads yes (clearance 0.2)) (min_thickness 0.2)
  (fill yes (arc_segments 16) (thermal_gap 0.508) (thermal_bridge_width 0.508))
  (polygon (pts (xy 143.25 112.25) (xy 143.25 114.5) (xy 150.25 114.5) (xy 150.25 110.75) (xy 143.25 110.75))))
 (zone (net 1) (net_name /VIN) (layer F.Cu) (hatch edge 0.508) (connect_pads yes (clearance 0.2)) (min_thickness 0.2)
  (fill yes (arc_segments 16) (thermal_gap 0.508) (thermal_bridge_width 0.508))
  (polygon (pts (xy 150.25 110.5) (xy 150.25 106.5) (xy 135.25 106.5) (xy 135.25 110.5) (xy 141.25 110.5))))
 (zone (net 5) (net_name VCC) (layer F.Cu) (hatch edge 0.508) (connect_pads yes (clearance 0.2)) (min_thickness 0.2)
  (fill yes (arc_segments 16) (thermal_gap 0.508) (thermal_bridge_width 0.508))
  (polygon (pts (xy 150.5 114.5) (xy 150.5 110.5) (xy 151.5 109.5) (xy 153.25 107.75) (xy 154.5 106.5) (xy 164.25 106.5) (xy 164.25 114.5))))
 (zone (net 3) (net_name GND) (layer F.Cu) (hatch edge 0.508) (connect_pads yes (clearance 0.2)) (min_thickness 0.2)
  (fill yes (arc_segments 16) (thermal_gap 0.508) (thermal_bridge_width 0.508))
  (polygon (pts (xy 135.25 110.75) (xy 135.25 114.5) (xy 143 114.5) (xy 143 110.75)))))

